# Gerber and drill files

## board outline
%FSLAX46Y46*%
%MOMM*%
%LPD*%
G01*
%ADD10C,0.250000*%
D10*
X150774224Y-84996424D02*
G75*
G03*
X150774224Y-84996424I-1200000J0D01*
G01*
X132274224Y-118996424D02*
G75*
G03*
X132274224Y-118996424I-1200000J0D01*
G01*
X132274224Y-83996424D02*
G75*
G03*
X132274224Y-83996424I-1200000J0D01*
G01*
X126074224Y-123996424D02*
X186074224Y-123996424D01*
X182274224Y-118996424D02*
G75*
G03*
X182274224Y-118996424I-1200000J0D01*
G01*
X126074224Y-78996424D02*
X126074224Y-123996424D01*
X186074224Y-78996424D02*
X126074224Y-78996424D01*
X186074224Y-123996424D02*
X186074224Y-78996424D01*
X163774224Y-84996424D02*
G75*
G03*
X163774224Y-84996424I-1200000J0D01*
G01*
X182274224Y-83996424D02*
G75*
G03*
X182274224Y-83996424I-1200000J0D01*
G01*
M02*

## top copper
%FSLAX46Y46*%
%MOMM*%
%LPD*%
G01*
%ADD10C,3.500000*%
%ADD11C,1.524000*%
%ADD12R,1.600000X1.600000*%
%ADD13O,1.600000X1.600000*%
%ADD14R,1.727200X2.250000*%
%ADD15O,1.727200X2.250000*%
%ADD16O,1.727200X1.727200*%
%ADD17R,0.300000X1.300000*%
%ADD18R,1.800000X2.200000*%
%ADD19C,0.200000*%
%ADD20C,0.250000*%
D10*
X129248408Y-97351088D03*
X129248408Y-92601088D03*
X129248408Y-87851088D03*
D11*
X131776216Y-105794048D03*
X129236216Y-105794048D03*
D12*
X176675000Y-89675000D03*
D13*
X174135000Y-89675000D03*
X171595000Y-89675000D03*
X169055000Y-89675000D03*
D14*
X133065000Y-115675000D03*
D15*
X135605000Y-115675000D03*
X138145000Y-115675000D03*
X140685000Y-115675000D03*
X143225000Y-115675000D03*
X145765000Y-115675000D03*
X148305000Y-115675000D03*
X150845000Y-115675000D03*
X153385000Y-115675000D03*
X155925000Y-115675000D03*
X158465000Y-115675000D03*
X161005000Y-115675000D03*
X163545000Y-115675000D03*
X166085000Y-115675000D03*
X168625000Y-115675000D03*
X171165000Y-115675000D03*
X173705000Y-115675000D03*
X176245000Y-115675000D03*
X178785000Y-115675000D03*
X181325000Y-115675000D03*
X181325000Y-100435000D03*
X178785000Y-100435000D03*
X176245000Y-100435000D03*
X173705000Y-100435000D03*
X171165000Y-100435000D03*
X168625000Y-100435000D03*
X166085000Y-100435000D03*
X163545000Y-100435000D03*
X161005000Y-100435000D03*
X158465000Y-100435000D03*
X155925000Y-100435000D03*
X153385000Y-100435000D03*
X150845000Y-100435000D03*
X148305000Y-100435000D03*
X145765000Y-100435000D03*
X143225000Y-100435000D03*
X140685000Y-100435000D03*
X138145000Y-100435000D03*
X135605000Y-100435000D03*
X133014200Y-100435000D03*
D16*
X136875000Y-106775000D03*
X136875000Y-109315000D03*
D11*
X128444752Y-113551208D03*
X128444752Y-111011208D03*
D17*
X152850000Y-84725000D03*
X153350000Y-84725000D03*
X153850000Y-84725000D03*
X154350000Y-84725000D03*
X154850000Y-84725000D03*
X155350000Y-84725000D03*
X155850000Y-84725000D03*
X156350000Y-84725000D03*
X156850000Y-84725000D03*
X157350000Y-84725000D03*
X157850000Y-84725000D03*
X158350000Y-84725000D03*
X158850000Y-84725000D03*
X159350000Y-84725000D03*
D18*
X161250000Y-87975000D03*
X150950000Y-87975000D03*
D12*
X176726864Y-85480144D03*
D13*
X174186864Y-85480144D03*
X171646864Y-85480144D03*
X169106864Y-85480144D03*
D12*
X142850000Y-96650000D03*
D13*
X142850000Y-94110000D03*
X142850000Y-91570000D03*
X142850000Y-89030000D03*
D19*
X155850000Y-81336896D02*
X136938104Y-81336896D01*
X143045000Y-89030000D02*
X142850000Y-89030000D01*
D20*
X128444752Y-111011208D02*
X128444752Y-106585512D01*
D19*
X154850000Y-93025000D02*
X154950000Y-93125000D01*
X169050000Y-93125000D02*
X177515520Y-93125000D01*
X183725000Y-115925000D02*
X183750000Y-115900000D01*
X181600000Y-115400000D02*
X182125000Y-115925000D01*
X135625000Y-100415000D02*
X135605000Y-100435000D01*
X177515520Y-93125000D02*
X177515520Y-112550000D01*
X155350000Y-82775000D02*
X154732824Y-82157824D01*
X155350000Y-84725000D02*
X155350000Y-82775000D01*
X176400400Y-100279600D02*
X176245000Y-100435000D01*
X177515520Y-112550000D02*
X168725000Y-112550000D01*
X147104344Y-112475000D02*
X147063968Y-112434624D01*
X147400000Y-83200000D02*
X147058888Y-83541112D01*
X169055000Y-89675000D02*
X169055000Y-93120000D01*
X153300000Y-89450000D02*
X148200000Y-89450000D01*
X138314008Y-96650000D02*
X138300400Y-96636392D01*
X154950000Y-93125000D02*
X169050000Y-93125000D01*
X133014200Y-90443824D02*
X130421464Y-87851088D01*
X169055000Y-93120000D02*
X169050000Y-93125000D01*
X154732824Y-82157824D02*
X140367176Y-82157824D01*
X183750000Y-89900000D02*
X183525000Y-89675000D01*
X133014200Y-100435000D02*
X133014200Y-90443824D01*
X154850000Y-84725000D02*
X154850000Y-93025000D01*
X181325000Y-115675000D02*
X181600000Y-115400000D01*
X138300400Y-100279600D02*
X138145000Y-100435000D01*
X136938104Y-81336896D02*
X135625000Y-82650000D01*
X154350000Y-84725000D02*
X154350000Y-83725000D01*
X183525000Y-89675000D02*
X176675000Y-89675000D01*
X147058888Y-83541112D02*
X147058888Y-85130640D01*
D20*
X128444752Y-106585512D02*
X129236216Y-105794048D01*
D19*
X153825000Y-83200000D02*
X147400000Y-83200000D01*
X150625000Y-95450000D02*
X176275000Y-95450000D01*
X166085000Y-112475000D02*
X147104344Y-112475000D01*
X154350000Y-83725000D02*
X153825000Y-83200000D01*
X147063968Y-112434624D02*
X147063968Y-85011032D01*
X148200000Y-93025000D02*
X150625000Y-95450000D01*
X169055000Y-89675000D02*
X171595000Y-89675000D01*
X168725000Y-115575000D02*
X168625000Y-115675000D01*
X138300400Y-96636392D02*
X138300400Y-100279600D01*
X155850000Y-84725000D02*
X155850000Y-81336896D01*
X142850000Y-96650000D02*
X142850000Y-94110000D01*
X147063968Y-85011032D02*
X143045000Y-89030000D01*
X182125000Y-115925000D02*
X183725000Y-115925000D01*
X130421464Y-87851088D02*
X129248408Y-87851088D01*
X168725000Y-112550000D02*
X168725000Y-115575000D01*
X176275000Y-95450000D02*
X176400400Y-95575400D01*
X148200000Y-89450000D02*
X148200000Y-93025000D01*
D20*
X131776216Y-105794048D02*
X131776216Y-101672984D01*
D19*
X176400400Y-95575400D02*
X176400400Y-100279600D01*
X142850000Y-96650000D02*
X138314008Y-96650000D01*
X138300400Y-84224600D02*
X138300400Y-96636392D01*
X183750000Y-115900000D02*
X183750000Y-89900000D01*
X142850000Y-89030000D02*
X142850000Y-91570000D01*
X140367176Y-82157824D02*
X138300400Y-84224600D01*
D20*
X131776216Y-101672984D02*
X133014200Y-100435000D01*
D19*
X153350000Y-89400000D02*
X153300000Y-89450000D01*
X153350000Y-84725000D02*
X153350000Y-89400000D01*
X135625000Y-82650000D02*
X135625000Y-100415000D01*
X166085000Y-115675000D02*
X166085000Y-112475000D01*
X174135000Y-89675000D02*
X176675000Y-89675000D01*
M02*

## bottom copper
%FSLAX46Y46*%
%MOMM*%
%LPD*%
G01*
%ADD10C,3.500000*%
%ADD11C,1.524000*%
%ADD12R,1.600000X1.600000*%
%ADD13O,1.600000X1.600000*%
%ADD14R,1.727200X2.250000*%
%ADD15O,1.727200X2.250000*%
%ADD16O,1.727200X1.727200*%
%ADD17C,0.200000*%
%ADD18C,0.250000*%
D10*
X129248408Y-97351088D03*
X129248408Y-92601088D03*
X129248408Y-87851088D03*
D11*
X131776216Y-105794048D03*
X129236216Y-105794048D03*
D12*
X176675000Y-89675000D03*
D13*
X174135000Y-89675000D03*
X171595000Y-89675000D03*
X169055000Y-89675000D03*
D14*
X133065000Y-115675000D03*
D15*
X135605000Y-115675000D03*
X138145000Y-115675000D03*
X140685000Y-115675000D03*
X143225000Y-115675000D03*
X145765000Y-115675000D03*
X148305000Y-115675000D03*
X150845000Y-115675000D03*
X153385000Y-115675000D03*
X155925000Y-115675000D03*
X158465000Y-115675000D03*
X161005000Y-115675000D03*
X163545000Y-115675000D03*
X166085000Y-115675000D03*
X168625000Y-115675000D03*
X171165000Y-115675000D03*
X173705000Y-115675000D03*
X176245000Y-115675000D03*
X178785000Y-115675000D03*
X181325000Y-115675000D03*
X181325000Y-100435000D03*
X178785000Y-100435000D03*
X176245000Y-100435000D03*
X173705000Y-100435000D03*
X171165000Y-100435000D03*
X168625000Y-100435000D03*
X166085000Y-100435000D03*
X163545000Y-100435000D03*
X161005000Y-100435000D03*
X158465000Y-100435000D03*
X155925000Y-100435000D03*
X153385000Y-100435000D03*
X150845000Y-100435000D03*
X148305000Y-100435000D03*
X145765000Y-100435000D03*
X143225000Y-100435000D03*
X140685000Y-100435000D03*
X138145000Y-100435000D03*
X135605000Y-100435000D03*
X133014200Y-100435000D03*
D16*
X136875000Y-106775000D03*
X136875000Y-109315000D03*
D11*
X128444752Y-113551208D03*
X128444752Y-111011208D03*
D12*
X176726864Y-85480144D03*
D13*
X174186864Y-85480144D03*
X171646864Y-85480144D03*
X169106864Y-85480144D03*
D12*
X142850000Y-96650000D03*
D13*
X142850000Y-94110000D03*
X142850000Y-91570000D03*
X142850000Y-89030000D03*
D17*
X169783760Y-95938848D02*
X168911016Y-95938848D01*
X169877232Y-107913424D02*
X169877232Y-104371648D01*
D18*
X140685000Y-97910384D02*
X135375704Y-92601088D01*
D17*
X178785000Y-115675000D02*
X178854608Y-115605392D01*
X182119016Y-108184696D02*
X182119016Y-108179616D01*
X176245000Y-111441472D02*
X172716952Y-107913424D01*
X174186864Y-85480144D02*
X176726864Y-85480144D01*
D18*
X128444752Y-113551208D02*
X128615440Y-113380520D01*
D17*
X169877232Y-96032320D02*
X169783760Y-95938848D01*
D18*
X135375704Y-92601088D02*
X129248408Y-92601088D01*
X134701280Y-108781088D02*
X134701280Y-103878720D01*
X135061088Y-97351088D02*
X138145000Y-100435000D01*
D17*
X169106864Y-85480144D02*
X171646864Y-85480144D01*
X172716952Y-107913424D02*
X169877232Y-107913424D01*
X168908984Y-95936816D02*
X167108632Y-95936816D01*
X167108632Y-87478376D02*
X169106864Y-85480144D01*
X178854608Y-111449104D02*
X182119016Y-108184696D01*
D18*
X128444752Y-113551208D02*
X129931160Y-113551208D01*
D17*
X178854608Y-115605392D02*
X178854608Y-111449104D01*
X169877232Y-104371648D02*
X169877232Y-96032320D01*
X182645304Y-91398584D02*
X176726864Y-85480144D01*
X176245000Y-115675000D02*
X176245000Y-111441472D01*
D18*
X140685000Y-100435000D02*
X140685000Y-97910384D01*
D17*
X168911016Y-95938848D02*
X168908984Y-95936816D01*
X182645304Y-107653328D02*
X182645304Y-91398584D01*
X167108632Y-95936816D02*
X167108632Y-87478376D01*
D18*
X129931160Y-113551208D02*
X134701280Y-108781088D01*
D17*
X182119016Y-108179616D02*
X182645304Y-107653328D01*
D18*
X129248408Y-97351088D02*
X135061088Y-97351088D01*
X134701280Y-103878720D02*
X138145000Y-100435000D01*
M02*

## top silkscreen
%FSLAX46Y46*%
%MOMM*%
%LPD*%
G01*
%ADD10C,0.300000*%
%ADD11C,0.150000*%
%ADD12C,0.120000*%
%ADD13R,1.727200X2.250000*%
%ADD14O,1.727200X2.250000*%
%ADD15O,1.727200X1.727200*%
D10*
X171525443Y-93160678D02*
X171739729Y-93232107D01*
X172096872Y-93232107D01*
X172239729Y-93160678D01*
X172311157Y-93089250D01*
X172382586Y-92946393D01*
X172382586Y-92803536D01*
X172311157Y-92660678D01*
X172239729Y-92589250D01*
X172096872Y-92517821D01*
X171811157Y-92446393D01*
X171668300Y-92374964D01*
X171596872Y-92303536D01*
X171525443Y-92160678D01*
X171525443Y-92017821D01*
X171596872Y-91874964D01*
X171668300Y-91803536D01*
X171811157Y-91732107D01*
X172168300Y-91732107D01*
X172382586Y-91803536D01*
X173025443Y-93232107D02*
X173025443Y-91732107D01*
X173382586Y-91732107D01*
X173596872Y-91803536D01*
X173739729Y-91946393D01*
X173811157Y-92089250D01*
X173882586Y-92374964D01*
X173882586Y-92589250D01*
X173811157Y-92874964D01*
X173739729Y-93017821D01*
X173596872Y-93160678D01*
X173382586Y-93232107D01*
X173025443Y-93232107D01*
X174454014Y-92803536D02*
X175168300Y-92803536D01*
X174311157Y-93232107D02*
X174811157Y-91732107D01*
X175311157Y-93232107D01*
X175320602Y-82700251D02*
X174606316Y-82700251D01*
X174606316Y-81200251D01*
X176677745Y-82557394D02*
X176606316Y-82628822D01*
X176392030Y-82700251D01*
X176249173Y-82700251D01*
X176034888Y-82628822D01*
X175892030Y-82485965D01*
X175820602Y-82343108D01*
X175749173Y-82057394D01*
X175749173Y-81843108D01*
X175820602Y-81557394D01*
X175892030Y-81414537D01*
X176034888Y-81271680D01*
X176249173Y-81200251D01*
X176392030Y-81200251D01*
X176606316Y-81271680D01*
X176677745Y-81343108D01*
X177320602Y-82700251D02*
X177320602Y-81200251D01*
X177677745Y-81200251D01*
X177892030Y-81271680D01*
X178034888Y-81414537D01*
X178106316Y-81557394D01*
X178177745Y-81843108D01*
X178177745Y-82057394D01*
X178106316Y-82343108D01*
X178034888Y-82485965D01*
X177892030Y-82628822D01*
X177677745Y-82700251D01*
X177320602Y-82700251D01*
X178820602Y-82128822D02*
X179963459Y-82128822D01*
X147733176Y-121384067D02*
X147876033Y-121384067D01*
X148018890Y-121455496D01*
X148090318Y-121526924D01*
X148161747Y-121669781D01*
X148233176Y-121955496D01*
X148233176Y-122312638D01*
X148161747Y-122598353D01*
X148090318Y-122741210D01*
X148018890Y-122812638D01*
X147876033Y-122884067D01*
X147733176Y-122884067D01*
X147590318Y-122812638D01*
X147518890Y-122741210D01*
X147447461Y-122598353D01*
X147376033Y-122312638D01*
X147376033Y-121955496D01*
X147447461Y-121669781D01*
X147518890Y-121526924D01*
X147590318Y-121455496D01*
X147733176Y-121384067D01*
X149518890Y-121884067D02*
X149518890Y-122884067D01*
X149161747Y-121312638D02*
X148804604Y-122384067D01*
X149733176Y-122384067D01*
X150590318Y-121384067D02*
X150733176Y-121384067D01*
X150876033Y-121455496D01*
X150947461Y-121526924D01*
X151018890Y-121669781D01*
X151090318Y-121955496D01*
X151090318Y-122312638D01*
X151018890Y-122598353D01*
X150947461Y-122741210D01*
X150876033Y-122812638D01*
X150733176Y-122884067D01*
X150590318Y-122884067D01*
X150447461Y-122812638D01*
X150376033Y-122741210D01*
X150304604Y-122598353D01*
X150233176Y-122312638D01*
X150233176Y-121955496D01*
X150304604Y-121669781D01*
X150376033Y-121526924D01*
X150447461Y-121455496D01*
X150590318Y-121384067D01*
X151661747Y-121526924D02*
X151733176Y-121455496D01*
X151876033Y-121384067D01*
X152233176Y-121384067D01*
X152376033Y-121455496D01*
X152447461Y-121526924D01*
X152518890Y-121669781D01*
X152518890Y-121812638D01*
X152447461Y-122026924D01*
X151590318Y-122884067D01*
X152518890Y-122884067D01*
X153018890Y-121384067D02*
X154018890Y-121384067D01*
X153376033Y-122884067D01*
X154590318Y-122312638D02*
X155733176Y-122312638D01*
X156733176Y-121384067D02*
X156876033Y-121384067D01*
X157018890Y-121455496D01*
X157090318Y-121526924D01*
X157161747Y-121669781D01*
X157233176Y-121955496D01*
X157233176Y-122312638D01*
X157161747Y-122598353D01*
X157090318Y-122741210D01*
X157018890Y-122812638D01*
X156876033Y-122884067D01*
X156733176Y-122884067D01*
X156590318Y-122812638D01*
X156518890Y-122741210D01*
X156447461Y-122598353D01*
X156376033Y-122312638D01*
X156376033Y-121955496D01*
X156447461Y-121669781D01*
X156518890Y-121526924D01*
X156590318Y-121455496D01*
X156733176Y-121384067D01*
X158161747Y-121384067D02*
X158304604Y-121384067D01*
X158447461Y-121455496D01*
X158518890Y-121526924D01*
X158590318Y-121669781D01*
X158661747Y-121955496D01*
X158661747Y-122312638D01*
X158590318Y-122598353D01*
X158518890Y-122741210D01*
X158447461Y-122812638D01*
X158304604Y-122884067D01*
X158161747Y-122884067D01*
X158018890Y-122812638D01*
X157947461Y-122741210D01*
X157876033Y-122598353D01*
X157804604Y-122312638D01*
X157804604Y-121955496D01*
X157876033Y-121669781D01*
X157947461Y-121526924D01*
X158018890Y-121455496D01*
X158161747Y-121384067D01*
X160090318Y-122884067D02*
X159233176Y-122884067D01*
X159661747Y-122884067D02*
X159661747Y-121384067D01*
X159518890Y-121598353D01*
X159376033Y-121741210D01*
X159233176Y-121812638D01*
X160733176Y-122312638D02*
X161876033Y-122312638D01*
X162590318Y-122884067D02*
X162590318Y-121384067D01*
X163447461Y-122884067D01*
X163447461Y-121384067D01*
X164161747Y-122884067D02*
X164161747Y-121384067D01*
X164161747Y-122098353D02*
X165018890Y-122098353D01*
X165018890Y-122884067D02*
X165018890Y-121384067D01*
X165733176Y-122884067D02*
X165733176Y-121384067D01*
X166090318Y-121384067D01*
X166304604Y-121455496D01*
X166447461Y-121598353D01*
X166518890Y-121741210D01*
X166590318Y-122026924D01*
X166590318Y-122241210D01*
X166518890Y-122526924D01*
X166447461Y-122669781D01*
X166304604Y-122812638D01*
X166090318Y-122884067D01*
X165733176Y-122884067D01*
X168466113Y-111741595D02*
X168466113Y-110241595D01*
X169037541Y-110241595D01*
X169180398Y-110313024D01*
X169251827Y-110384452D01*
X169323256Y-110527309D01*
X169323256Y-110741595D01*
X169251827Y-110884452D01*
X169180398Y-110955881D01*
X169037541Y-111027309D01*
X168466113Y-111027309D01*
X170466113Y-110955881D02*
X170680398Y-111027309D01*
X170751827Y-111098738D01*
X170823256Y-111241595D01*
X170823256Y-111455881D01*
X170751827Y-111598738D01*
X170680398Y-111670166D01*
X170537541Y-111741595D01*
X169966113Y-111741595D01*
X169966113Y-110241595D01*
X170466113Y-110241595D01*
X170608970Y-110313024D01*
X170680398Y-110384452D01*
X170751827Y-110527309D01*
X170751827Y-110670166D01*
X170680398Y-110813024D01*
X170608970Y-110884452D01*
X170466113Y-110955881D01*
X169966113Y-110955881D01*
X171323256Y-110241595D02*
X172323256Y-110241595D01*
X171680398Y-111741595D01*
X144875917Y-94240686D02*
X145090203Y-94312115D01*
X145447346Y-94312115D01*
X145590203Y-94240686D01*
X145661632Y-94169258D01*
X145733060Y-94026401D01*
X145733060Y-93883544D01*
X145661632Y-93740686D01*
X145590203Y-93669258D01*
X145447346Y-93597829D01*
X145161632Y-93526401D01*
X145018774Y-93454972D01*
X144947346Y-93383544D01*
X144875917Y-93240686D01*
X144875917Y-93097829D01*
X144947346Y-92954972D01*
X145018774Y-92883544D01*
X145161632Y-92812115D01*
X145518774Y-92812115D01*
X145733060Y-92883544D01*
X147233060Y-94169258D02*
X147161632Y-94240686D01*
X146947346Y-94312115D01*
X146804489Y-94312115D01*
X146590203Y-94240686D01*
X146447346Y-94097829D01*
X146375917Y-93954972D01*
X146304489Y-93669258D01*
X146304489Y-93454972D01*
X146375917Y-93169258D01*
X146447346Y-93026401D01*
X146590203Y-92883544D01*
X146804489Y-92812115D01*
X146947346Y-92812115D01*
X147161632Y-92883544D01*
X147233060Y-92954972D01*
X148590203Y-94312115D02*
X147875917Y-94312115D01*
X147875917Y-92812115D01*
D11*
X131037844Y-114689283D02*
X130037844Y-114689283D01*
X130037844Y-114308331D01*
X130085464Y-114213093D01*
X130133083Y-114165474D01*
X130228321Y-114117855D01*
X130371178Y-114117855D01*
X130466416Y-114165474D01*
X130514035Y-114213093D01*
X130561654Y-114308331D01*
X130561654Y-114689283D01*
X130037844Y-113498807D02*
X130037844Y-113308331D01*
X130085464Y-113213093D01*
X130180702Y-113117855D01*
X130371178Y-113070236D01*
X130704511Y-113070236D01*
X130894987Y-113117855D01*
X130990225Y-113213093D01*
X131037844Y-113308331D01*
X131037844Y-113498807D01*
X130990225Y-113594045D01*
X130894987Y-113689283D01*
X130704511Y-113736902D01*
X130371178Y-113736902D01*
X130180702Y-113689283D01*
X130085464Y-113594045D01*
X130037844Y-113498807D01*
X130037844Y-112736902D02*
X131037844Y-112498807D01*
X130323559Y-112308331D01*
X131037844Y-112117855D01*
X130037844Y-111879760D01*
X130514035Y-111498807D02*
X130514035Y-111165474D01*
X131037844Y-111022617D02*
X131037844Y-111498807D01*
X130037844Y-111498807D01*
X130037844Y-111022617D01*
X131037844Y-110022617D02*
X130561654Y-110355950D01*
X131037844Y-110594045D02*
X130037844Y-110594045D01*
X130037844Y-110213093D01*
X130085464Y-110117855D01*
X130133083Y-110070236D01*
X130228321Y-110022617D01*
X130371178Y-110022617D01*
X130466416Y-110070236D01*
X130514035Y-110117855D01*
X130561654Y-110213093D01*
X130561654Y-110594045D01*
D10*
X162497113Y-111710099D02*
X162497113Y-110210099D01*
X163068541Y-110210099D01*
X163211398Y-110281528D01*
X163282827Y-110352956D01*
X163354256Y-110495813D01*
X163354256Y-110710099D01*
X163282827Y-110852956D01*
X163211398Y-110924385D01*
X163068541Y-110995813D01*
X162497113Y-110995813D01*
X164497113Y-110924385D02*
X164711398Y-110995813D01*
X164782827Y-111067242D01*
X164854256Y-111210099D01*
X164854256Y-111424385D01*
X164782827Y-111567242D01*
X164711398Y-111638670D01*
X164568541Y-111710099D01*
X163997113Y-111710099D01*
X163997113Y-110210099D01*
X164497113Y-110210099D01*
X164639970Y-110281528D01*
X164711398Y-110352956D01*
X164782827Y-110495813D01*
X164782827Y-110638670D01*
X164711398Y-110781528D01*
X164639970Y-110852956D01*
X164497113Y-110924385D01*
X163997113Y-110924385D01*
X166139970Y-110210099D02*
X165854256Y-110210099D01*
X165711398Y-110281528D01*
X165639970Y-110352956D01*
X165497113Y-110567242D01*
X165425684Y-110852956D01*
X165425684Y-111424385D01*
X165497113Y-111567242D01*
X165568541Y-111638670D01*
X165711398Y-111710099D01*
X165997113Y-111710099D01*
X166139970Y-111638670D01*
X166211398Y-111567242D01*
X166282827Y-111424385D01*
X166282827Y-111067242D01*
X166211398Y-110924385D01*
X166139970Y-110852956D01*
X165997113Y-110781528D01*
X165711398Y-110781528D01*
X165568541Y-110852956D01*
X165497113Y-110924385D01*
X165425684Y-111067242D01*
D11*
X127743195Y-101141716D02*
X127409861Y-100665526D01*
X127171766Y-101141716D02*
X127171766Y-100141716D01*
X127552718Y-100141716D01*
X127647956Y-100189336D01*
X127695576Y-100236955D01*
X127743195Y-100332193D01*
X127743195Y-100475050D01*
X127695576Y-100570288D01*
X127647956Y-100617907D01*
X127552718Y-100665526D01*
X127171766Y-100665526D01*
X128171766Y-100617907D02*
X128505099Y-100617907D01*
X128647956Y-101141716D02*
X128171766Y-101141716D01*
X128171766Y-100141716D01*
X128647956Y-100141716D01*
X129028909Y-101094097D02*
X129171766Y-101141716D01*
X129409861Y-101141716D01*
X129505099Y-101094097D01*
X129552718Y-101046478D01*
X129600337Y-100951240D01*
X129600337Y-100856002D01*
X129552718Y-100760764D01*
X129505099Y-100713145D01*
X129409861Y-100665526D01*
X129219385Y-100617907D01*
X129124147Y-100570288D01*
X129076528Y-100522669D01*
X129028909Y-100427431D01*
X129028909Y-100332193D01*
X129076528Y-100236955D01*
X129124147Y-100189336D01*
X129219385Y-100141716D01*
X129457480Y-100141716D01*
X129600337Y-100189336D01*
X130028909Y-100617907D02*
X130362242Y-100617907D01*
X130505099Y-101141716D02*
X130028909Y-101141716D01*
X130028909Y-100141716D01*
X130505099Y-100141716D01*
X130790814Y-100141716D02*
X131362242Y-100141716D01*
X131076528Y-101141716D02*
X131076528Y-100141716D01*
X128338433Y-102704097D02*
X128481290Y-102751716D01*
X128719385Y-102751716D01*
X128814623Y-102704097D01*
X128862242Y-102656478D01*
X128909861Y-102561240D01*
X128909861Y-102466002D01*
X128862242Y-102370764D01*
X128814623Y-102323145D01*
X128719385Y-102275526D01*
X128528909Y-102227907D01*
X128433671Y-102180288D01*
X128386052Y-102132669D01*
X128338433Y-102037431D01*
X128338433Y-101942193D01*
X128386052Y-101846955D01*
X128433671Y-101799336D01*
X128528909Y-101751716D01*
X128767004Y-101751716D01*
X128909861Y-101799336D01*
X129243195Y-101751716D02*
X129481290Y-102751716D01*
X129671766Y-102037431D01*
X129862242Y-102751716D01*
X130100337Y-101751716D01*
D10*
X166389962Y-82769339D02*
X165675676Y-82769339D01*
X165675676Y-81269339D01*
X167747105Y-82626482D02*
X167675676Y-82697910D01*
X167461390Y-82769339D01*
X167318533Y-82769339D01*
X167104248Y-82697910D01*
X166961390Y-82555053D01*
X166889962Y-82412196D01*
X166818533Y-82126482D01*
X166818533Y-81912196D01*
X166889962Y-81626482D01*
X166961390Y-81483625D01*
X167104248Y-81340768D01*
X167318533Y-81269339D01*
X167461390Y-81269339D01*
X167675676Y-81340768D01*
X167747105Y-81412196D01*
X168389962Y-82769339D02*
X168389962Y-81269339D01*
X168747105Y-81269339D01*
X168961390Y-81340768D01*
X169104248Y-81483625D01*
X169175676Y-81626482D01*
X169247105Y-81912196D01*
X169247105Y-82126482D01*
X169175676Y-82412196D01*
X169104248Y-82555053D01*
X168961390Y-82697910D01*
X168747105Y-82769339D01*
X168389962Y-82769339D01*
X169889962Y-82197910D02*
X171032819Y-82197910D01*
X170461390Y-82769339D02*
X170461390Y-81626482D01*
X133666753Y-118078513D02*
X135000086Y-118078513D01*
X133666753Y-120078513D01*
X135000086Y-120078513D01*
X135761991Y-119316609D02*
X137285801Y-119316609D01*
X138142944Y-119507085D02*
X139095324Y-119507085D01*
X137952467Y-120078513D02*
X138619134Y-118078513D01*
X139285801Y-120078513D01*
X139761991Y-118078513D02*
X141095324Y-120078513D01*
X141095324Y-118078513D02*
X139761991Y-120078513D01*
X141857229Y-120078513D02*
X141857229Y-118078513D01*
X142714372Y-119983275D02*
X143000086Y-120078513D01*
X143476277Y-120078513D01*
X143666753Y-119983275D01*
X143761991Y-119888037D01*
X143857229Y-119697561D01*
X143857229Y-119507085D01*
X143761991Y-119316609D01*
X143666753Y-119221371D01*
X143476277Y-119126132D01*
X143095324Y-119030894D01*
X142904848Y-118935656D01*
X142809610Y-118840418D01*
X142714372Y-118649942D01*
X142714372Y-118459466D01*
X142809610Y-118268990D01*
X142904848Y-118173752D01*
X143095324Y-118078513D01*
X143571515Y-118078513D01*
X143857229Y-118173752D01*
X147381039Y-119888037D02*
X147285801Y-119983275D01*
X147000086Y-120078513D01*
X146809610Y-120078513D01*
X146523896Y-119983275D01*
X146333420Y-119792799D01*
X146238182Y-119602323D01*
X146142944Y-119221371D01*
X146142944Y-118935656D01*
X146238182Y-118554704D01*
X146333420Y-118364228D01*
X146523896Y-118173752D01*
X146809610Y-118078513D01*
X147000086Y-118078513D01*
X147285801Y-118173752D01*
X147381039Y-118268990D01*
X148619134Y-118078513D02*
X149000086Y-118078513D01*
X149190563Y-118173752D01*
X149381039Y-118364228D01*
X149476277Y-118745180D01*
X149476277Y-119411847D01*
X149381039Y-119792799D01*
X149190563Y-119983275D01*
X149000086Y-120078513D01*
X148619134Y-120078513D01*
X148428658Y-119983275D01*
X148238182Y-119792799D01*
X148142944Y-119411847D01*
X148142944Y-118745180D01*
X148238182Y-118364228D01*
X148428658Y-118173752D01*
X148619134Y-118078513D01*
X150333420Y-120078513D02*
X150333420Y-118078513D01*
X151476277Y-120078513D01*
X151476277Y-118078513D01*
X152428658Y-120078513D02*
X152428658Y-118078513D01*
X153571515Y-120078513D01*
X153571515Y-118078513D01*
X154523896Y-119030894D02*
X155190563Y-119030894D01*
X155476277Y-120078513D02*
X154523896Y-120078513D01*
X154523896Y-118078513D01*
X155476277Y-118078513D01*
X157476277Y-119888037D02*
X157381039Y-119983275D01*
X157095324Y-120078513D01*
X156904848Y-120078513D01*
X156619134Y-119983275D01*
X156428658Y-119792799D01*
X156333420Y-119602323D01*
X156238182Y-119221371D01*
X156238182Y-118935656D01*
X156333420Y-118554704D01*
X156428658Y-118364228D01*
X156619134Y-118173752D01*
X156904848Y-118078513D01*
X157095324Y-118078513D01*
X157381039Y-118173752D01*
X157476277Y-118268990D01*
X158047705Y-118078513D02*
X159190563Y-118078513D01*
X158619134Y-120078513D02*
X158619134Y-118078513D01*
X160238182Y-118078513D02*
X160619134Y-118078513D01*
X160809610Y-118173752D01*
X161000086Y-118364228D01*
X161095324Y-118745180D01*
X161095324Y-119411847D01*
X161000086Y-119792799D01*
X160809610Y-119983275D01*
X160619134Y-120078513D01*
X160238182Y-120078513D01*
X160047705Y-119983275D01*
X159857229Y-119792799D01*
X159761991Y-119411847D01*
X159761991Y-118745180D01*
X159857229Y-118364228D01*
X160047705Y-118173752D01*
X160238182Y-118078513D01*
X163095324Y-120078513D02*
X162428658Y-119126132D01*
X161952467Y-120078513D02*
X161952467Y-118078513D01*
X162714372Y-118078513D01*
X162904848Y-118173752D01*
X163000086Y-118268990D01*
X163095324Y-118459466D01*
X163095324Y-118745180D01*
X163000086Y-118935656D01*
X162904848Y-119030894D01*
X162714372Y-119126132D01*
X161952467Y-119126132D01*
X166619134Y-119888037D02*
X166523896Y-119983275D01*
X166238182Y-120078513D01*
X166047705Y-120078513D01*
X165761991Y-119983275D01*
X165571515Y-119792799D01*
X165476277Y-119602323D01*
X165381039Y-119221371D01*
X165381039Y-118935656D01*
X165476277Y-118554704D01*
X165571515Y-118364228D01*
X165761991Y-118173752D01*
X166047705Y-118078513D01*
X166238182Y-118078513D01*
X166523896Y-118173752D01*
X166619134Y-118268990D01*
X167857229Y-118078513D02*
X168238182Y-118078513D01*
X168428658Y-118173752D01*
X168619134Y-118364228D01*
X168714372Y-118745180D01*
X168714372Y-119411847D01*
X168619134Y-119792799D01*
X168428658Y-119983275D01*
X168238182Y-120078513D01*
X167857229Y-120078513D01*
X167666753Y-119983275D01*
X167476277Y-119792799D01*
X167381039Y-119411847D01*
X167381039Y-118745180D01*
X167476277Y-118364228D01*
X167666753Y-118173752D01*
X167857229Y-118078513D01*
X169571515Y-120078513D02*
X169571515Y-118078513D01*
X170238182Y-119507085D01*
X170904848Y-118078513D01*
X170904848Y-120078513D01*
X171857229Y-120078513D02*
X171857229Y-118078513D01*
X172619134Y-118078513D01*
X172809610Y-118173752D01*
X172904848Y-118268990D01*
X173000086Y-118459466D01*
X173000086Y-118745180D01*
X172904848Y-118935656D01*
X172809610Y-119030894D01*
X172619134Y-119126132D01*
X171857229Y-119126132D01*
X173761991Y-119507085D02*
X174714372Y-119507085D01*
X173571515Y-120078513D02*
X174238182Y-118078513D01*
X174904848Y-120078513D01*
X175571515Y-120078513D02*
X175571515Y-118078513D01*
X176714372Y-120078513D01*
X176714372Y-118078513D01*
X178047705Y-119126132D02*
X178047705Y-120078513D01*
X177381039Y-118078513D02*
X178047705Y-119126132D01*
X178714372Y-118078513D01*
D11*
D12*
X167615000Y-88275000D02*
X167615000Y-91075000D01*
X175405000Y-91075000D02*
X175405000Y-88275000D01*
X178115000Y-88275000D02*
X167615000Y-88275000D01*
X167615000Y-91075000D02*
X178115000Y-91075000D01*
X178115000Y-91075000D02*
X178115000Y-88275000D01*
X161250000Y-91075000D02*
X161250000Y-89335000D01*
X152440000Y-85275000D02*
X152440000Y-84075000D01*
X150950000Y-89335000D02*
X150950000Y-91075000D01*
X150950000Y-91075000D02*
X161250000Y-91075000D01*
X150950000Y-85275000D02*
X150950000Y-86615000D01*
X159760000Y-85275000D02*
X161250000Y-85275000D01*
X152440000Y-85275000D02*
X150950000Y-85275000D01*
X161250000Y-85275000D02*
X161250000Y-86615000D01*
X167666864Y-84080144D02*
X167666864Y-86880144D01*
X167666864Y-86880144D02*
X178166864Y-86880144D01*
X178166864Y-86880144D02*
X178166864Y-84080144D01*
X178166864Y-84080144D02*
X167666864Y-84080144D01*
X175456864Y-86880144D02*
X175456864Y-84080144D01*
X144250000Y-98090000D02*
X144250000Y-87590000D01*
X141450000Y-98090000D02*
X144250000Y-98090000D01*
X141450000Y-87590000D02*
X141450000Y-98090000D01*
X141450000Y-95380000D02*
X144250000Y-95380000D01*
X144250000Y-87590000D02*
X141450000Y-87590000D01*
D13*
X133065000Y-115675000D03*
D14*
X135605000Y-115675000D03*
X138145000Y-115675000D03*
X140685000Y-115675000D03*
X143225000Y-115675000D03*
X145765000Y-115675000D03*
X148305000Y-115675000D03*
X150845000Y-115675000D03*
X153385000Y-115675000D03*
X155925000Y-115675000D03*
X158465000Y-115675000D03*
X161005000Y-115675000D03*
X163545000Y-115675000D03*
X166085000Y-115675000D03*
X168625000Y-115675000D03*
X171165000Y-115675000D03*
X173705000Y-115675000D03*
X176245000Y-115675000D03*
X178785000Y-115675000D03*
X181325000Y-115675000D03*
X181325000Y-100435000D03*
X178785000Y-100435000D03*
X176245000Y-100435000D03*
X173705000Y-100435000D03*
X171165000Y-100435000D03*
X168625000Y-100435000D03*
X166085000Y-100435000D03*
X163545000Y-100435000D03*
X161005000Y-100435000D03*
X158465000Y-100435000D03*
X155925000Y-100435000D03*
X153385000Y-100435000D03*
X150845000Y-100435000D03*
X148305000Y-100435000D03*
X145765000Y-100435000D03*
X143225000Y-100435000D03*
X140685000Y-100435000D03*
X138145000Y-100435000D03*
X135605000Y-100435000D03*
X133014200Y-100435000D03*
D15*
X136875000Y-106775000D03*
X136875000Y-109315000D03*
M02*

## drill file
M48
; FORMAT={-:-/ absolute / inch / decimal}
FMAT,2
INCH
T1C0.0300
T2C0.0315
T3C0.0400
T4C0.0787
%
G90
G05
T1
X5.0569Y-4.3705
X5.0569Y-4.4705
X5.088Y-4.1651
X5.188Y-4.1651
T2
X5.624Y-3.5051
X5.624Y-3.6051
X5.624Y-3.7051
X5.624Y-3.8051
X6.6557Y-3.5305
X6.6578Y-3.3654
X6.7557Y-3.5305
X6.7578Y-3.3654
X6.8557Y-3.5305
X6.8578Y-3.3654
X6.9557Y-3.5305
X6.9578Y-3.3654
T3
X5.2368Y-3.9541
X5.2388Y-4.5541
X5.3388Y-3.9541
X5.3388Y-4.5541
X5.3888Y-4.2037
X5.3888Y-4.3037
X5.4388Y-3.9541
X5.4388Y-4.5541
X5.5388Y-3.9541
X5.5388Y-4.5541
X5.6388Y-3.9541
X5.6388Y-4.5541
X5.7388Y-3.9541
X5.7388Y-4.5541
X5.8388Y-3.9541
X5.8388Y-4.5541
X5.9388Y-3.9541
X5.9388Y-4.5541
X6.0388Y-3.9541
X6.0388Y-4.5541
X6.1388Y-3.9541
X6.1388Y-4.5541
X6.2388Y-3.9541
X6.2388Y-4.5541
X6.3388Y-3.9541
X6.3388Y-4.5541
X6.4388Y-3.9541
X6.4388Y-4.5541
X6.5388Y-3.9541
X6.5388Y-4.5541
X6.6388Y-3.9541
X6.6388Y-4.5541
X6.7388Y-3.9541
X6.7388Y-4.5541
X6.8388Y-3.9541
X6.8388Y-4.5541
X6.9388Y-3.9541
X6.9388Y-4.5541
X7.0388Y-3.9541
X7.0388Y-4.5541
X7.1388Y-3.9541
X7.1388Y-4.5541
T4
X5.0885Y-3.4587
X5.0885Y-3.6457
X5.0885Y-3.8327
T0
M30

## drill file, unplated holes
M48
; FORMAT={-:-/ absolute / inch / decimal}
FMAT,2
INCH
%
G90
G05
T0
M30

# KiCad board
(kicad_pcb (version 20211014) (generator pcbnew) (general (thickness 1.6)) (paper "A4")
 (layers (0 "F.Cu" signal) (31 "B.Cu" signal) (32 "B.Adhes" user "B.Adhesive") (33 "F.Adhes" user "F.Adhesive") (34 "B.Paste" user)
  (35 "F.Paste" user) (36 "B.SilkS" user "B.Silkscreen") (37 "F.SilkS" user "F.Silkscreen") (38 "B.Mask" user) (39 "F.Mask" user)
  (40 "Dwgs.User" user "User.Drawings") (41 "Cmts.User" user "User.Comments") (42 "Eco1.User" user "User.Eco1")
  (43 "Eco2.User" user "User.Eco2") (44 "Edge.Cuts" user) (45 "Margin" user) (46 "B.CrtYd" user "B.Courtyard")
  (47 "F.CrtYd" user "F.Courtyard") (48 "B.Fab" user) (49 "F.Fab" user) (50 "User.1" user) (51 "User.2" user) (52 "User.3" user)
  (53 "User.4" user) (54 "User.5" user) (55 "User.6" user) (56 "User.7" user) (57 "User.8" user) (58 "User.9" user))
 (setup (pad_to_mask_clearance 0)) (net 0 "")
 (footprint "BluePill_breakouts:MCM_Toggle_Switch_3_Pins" (layer "F.Cu") (at 129.248408 97.351088 90)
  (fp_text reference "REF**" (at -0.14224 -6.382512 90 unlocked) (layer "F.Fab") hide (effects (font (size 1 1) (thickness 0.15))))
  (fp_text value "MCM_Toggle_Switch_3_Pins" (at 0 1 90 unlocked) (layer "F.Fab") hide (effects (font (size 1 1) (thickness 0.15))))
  (pad "1" thru_hole circle (at 0 0 90) (size 3.5 3.5) (drill 2) (layers *.Cu *.Mask))
  (pad "2" thru_hole circle (at 4.75 0 90) (size 3.5 3.5) (drill 2) (layers *.Cu *.Mask))
  (pad "3" thru_hole circle (at 9.5 0 90) (size 3.5 3.5) (drill 2) (layers *.Cu *.Mask)))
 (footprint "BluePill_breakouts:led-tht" (layer "F.Cu") (at 131.776216 105.794048 180)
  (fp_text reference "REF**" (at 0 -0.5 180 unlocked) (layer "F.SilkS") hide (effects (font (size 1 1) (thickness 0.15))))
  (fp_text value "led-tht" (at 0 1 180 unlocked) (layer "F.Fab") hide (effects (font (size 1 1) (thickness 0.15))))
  (pad "1" thru_hole circle (at 0 0 180) (size 1.524 1.524) (drill 0.762) (layers *.Cu *.Mask))
  (pad "2" thru_hole circle (at 2.54 0 180) (size 1.524 1.524) (drill 0.762) (layers *.Cu *.Mask)))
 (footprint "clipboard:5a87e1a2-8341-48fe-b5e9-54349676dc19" (layer "F.Cu") (at 176.675 89.675 180)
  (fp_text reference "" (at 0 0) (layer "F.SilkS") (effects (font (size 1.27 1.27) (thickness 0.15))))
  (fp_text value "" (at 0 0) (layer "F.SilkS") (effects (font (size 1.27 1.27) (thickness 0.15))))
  (fp_line (start 9.06 1.4) (end 9.06 -1.4) (layer "F.SilkS") (width 0.12))
  (fp_line (start 1.27 -1.4) (end 1.27 1.4) (layer "F.SilkS") (width 0.12))
  (fp_line (start -1.44 1.4) (end 9.06 1.4) (layer "F.SilkS") (width 0.12))
  (fp_line (start 9.06 -1.4) (end -1.44 -1.4) (layer "F.SilkS") (width 0.12))
  (fp_line (start -1.44 -1.4) (end -1.44 1.4) (layer "F.SilkS") (width 0.12))
  (pad "1" thru_hole rect (at 0 0 180) (size 1.6 1.6) (drill 0.8) (layers *.Cu *.Mask))
  (pad "2" thru_hole oval (at 2.54 0 180) (size 1.6 1.6) (drill 0.8) (layers *.Cu *.Mask))
  (pad "3" thru_hole oval (at 5.08 0 180) (size 1.6 1.6) (drill 0.8) (layers *.Cu *.Mask))
  (pad "4" thru_hole oval (at 7.62 0 180) (size 1.6 1.6) (drill 0.8) (layers *.Cu *.Mask)))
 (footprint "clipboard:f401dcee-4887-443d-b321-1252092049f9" (layer "F.Cu") (at 133.0142 100.435 90)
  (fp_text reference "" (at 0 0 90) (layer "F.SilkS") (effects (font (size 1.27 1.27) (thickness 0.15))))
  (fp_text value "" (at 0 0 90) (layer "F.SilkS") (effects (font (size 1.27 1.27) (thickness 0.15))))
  (pad "1" thru_hole rect (at -15.24 0.0508) (size 1.7272 2.25) (drill 1.016) (layers *.Cu *.Mask "F.SilkS"))
  (pad "2" thru_hole oval (at -15.24 2.5908) (size 1.7272 2.25) (drill 1.016) (layers *.Cu *.Mask "F.SilkS"))
  (pad "3" thru_hole oval (at -15.24 5.1308) (size 1.7272 2.25) (drill 1.016) (layers *.Cu *.Mask "F.SilkS"))
  (pad "4" thru_hole oval (at -15.24 7.6708) (size 1.7272 2.25) (drill 1.016) (layers *.Cu *.Mask "F.SilkS"))
  (pad "5" thru_hole oval (at -15.24 10.2108) (size 1.7272 2.25) (drill 1.016) (layers *.Cu *.Mask "F.SilkS"))
  (pad "6" thru_hole oval (at -15.24 12.7508) (size 1.7272 2.25) (drill 1.016) (layers *.Cu *.Mask "F.SilkS"))
  (pad "7" thru_hole oval (at -15.24 15.2908) (size 1.7272 2.25) (drill 1.016) (layers *.Cu *.Mask "F.SilkS"))
  (pad "8" thru_hole oval (at -15.24 17.8308) (size 1.7272 2.25) (drill 1.016) (layers *.Cu *.Mask "F.SilkS"))
  (pad "9" thru_hole oval (at -15.24 20.3708) (size 1.7272 2.25) (drill 1.016) (layers *.Cu *.Mask "F.SilkS"))
  (pad "10" thru_hole oval (at -15.24 22.9108) (size 1.7272 2.25) (drill 1.016) (layers *.Cu *.Mask "F.SilkS"))
  (pad "11" thru_hole oval (at -15.24 25.4508) (size 1.7272 2.25) (drill 1.016) (layers *.Cu *.Mask "F.SilkS"))
  (pad "12" thru_hole oval (at -15.24 27.9908) (size 1.7272 2.25) (drill 1.016) (layers *.Cu *.Mask "F.SilkS"))
  (pad "13" thru_hole oval (at -15.24 30.5308) (size 1.7272 2.25) (drill 1.016) (layers *.Cu *.Mask "F.SilkS"))
  (pad "14" thru_hole oval (at -15.24 33.0708) (size 1.7272 2.25) (drill 1.016) (layers *.Cu *.Mask "F.SilkS"))
  (pad "15" thru_hole oval (at -15.24 35.6108) (size 1.7272 2.25) (drill 1.016) (layers *.Cu *.Mask "F.SilkS"))
  (pad "16" thru_hole oval (at -15.24 38.1508) (size 1.7272 2.25) (drill 1.016) (layers *.Cu *.Mask "F.SilkS"))
  (pad "17" thru_hole oval (at -15.24 40.6908) (size 1.7272 2.25) (drill 1.016) (layers *.Cu *.Mask "F.SilkS"))
  (pad "18" thru_hole oval (at -15.24 43.2308) (size 1.7272 2.25) (drill 1.016) (layers *.Cu *.Mask "F.SilkS"))
  (pad "19" thru_hole oval (at -15.24 45.7708) (size 1.7272 2.25) (drill 1.016) (layers *.Cu *.Mask "F.SilkS"))
  (pad "20" thru_hole oval (at -15.24 48.3108) (size 1.7272 2.25) (drill 1.016) (layers *.Cu *.Mask "F.SilkS"))
  (pad "21" thru_hole oval (at 0 48.3108 180) (size 1.7272 2.25) (drill 1.016) (layers *.Cu *.Mask "F.SilkS"))
  (pad "22" thru_hole oval (at 0 45.7708 180) (size 1.7272 2.25) (drill 1.016) (layers *.Cu *.Mask "F.SilkS"))
  (pad "23" thru_hole oval (at 0 43.2308 180) (size 1.7272 2.25) (drill 1.016) (layers *.Cu *.Mask "F.SilkS"))
  (pad "24" thru_hole oval (at 0 40.6908 180) (size 1.7272 2.25) (drill 1.016) (layers *.Cu *.Mask "F.SilkS"))
  (pad "25" thru_hole oval (at 0 38.1508 180) (size 1.7272 2.25) (drill 1.016) (layers *.Cu *.Mask "F.SilkS"))
  (pad "26" thru_hole oval (at 0 35.6108 180) (size 1.7272 2.25) (drill 1.016) (layers *.Cu *.Mask "F.SilkS"))
  (pad "27" thru_hole oval (at 0 33.0708 180) (size 1.7272 2.25) (drill 1.016) (layers *.Cu *.Mask "F.SilkS"))
  (pad "28" thru_hole oval (at 0 30.5308 180) (size 1.7272 2.25) (drill 1.016) (layers *.Cu *.Mask "F.SilkS"))
  (pad "29" thru_hole oval (at 0 27.9908 180) (size 1.7272 2.25) (drill 1.016) (layers *.Cu *.Mask "F.SilkS"))
  (pad "30" thru_hole oval (at 0 25.4508 180) (size 1.7272 2.25) (drill 1.016) (layers *.Cu *.Mask "F.SilkS"))
  (pad "31" thru_hole oval (at 0 22.9108 180) (size 1.7272 2.25) (drill 1.016) (layers *.Cu *.Mask "F.SilkS"))
  (pad "32" thru_hole oval (at 0 20.3708 180) (size 1.7272 2.25) (drill 1.016) (layers *.Cu *.Mask "F.SilkS"))
  (pad "33" thru_hole oval (at 0 17.8308 180) (size 1.7272 2.25) (drill 1.016) (layers *.Cu *.Mask "F.SilkS"))
  (pad "34" thru_hole oval (at 0 15.2908 180) (size 1.7272 2.25) (drill 1.016) (layers *.Cu *.Mask "F.SilkS"))
  (pad "35" thru_hole oval (at 0 12.7508 180) (size 1.7272 2.25) (drill 1.016) (layers *.Cu *.Mask "F.SilkS"))
  (pad "36" thru_hole oval (at 0 10.2108 180) (size 1.7272 2.25) (drill 1.016) (layers *.Cu *.Mask "F.SilkS"))
  (pad "37" thru_hole oval (at 0 7.6708 180) (size 1.7272 2.25) (drill 1.016) (layers *.Cu *.Mask "F.SilkS"))
  (pad "38" thru_hole oval (at 0 5.1308 180) (size 1.7272 2.25) (drill 1.016) (layers *.Cu *.Mask "F.SilkS"))
  (pad "39" thru_hole oval (at 0 2.5908 180) (size 1.7272 2.25) (drill 1.016) (layers *.Cu *.Mask "F.SilkS"))
  (pad "40" thru_hole oval (at 0 0 180) (size 1.7272 2.25) (drill 1.016) (layers *.Cu *.Mask "F.SilkS"))
  (pad "41" thru_hole oval (at -6.34 3.8608 180) (size 1.7272 1.7272) (drill 1.016) (layers *.Cu *.Mask "F.SilkS"))
  (pad "42" thru_hole oval (at -8.88 3.8608 180) (size 1.7272 1.7272) (drill 1.016) (layers *.Cu *.Mask "F.SilkS")))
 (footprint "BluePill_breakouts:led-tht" (layer "F.Cu") (at 128.444752 113.551208 90)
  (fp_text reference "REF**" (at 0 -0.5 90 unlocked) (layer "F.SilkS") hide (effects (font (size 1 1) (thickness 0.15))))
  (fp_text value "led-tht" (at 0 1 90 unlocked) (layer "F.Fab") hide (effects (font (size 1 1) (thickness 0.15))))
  (pad "1" thru_hole circle (at 0 0 90) (size 1.524 1.524) (drill 0.762) (layers *.Cu *.Mask))
  (pad "2" thru_hole circle (at 2.54 0 90) (size 1.524 1.524) (drill 0.762) (layers *.Cu *.Mask)))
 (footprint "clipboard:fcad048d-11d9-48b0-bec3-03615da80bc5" (layer "F.Cu") (at 156.1 85.375)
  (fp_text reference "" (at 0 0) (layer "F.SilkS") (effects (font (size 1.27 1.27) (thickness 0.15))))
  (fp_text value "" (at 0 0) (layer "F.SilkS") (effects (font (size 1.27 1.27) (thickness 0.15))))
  (fp_line (start 5.15 5.7) (end 5.15 3.96) (layer "F.SilkS") (width 0.12))
  (fp_line (start -3.66 -0.1) (end -3.66 -1.3) (layer "F.SilkS") (width 0.12))
  (fp_line (start -5.15 3.96) (end -5.15 5.7) (layer "F.SilkS") (width 0.12))
  (fp_line (start -5.15 5.7) (end 5.15 5.7) (layer "F.SilkS") (width 0.12))
  (fp_line (start -5.15 -0.1) (end -5.15 1.24) (layer "F.SilkS") (width 0.12))
  (fp_line (start 3.66 -0.1) (end 5.15 -0.1) (layer "F.SilkS") (width 0.12))
  (fp_line (start -3.66 -0.1) (end -5.15 -0.1) (layer "F.SilkS") (width 0.12))
  (fp_line (start 5.15 -0.1) (end 5.15 1.24) (layer "F.SilkS") (width 0.12))
  (pad "1" smd rect (at -3.25 -0.65) (size 0.3 1.3) (layers "F.Cu" "F.Paste" "F.Mask"))
  (pad "2" smd rect (at -2.75 -0.65) (size 0.3 1.3) (layers "F.Cu" "F.Paste" "F.Mask"))
  (pad "3" smd rect (at -2.25 -0.65) (size 0.3 1.3) (layers "F.Cu" "F.Paste" "F.Mask"))
  (pad "4" smd rect (at -1.75 -0.65) (size 0.3 1.3) (layers "F.Cu" "F.Paste" "F.Mask"))
  (pad "5" smd rect (at -1.25 -0.65) (size 0.3 1.3) (layers "F.Cu" "F.Paste" "F.Mask"))
  (pad "6" smd rect (at -0.75 -0.65) (size 0.3 1.3) (layers "F.Cu" "F.Paste" "F.Mask"))
  (pad "7" smd rect (at -0.25 -0.65) (size 0.3 1.3) (layers "F.Cu" "F.Paste" "F.Mask"))
  (pad "8" smd rect (at 0.25 -0.65) (size 0.3 1.3) (layers "F.Cu" "F.Paste" "F.Mask"))
  (pad "9" smd rect (at 0.75 -0.65) (size 0.3 1.3) (layers "F.Cu" "F.Paste" "F.Mask"))
  (pad "10" smd rect (at 1.25 -0.65) (size 0.3 1.3) (layers "F.Cu" "F.Paste" "F.Mask"))
  (pad "11" smd rect (at 1.75 -0.65) (size 0.3 1.3) (layers "F.Cu" "F.Paste" "F.Mask"))
  (pad "12" smd rect (at 2.25 -0.65) (size 0.3 1.3) (layers "F.Cu" "F.Paste" "F.Mask"))
  (pad "13" smd rect (at 2.75 -0.65) (size 0.3 1.3) (layers "F.Cu" "F.Paste" "F.Mask"))
  (pad "14" smd rect (at 3.25 -0.65) (size 0.3 1.3) (layers "F.Cu" "F.Paste" "F.Mask"))
  (pad "MP" smd rect (at 5.15 2.6) (size 1.8 2.2) (layers "F.Cu" "F.Paste" "F.Mask"))
  (pad "MP" smd rect (at -5.15 2.6) (size 1.8 2.2) (layers "F.Cu" "F.Paste" "F.Mask")))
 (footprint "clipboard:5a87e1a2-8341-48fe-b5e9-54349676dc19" (layer "F.Cu") (at 176.726864 85.480144 180)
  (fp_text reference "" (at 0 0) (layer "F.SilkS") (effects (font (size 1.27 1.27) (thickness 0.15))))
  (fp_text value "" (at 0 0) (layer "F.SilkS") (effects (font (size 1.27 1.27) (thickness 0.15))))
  (fp_line (start 9.06 1.4) (end 9.06 -1.4) (layer "F.SilkS") (width 0.12))
  (fp_line (start 9.06 -1.4) (end -1.44 -1.4) (layer "F.SilkS") (width 0.12))
  (fp_line (start -1.44 -1.4) (end -1.44 1.4) (layer "F.SilkS") (width 0.12))
  (fp_line (start -1.44 1.4) (end 9.06 1.4) (layer "F.SilkS") (width 0.12))
  (fp_line (start 1.27 -1.4) (end 1.27 1.4) (layer "F.SilkS") (width 0.12))
  (pad "1" thru_hole rect (at 0 0 180) (size 1.6 1.6) (drill 0.8) (layers *.Cu *.Mask))
  (pad "2" thru_hole oval (at 2.54 0 180) (size 1.6 1.6) (drill 0.8) (layers *.Cu *.Mask))
  (pad "3" thru_hole oval (at 5.08 0 180) (size 1.6 1.6) (drill 0.8) (layers *.Cu *.Mask))
  (pad "4" thru_hole oval (at 7.62 0 180) (size 1.6 1.6) (drill 0.8) (layers *.Cu *.Mask)))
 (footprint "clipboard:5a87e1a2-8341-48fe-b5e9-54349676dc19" (layer "F.Cu") (at 142.85 96.65 90)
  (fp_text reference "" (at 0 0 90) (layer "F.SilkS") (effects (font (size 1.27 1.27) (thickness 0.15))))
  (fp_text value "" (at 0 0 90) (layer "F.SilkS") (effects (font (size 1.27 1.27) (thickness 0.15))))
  (fp_line (start -1.44 1.4) (end 9.06 1.4) (layer "F.SilkS") (width 0.12))
  (fp_line (start -1.44 -1.4) (end -1.44 1.4) (layer "F.SilkS") (width 0.12))
  (fp_line (start 9.06 -1.4) (end -1.44 -1.4) (layer "F.SilkS") (width 0.12))
  (fp_line (start 1.27 -1.4) (end 1.27 1.4) (layer "F.SilkS") (width 0.12))
  (fp_line (start 9.06 1.4) (end 9.06 -1.4) (layer "F.SilkS") (width 0.12))
  (pad "1" thru_hole rect (at 0 0 90) (size 1.6 1.6) (drill 0.8) (layers *.Cu *.Mask))
  (pad "2" thru_hole oval (at 2.54 0 90) (size 1.6 1.6) (drill 0.8) (layers *.Cu *.Mask))
  (pad "3" thru_hole oval (at 5.08 0 90) (size 1.6 1.6) (drill 0.8) (layers *.Cu *.Mask))
  (pad "4" thru_hole oval (at 7.62 0 90) (size 1.6 1.6) (drill 0.8) (layers *.Cu *.Mask)))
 (gr_circle (center 149.574224 84.996424) (end 150.774224 84.996424) (layer "Edge.Cuts") (width 0.25) (fill none))
 (gr_circle (center 131.074224 118.996424) (end 132.274224 118.996424) (layer "Edge.Cuts") (width 0.25) (fill none))
 (gr_circle (center 131.074224 83.996424) (end 132.274224 83.996424) (layer "Edge.Cuts") (width 0.25) (fill none))
 (gr_line (start 126.074224 123.996424) (end 186.074224 123.996424) (layer "Edge.Cuts") (width 0.25))
 (gr_circle (center 181.074224 118.996424) (end 182.274224 118.996424) (layer "Edge.Cuts") (width 0.25) (fill none))
 (gr_line (start 126.074224 78.996424) (end 126.074224 123.996424) (layer "Edge.Cuts") (width 0.25))
 (gr_line (start 186.074224 78.996424) (end 126.074224 78.996424) (layer "Edge.Cuts") (width 0.25))
 (gr_line (start 186.074224 123.996424) (end 186.074224 78.996424) (layer "Edge.Cuts") (width 0.25))
 (gr_circle (center 162.574224 84.996424) (end 163.774224 84.996424) (layer "Edge.Cuts") (width 0.25) (fill none))
 (gr_circle (center 181.074224 83.996424) (end 182.274224 83.996424) (layer "Edge.Cuts") (width 0.25) (fill none))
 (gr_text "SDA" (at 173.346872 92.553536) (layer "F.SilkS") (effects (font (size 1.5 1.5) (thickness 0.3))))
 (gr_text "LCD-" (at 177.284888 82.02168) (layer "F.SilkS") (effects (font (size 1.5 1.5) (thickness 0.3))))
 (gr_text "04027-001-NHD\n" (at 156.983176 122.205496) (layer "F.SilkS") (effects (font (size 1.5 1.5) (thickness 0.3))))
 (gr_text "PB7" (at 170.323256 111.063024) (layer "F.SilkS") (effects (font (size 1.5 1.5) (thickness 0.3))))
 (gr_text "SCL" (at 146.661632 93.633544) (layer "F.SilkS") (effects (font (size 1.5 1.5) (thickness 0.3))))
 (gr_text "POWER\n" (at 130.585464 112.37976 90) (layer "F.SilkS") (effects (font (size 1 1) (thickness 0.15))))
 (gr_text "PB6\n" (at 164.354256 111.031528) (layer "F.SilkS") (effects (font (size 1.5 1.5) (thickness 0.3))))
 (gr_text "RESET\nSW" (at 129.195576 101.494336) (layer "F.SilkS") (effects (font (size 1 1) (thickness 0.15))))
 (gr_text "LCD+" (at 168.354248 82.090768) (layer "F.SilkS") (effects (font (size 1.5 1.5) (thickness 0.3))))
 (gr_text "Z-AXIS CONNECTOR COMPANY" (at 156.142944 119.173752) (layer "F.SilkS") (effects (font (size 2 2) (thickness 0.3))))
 (segment (start 155.85 81.336896) (end 136.938104 81.336896) (width 0.2) (layer "F.Cu") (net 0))
 (segment (start 143.045 89.03) (end 142.85 89.03) (width 0.2) (layer "F.Cu") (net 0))
 (segment (start 128.444752 111.011208) (end 128.444752 106.585512) (width 0.25) (layer "F.Cu") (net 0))
 (segment (start 154.85 93.025) (end 154.95 93.125) (width 0.2) (layer "F.Cu") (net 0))
 (segment (start 169.05 93.125) (end 177.51552 93.125) (width 0.2) (layer "F.Cu") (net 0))
 (segment (start 183.725 115.925) (end 183.75 115.9) (width 0.2) (layer "F.Cu") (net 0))
 (segment (start 181.6 115.4) (end 182.125 115.925) (width 0.2) (layer "F.Cu") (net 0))
 (segment (start 135.625 100.415) (end 135.605 100.435) (width 0.2) (layer "F.Cu") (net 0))
 (segment (start 177.51552 93.125) (end 177.51552 112.55) (width 0.2) (layer "F.Cu") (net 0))
 (segment (start 155.35 82.775) (end 154.732824 82.157824) (width 0.2) (layer "F.Cu") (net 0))
 (segment (start 155.35 84.725) (end 155.35 82.775) (width 0.2) (layer "F.Cu") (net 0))
 (segment (start 176.4004 100.2796) (end 176.245 100.435) (width 0.2) (layer "F.Cu") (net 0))
 (segment (start 177.51552 112.55) (end 168.725 112.55) (width 0.2) (layer "F.Cu") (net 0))
 (segment (start 147.104344 112.475) (end 147.063968 112.434624) (width 0.2) (layer "F.Cu") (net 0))
 (segment (start 147.4 83.2) (end 147.058888 83.541112) (width 0.2) (layer "F.Cu") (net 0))
 (segment (start 169.055 89.675) (end 169.055 93.12) (width 0.2) (layer "F.Cu") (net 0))
 (segment (start 153.3 89.45) (end 148.2 89.45) (width 0.2) (layer "F.Cu") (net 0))
 (segment (start 138.314008 96.65) (end 138.3004 96.636392) (width 0.2) (layer "F.Cu") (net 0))
 (segment (start 154.95 93.125) (end 169.05 93.125) (width 0.2) (layer "F.Cu") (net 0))
 (segment (start 133.0142 90.443824) (end 130.421464 87.851088) (width 0.2) (layer "F.Cu") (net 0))
 (segment (start 169.055 93.12) (end 169.05 93.125) (width 0.2) (layer "F.Cu") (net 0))
 (segment (start 154.732824 82.157824) (end 140.367176 82.157824) (width 0.2) (layer "F.Cu") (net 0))
 (segment (start 183.75 89.9) (end 183.525 89.675) (width 0.2) (layer "F.Cu") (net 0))
 (segment (start 133.0142 100.435) (end 133.0142 90.443824) (width 0.2) (layer "F.Cu") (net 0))
 (segment (start 154.85 84.725) (end 154.85 93.025) (width 0.2) (layer "F.Cu") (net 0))
 (segment (start 181.325 115.675) (end 181.6 115.4) (width 0.2) (layer "F.Cu") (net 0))
 (segment (start 138.3004 100.2796) (end 138.145 100.435) (width 0.2) (layer "F.Cu") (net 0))
 (segment (start 136.938104 81.336896) (end 135.625 82.65) (width 0.2) (layer "F.Cu") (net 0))
 (segment (start 154.35 84.725) (end 154.35 83.725) (width 0.2) (layer "F.Cu") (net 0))
 (segment (start 183.525 89.675) (end 176.675 89.675) (width 0.2) (layer "F.Cu") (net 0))
 (segment (start 147.058888 83.541112) (end 147.058888 85.13064) (width 0.2) (layer "F.Cu") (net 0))
 (segment (start 128.444752 106.585512) (end 129.236216 105.794048) (width 0.25) (layer "F.Cu") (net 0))
 (segment (start 153.825 83.2) (end 147.4 83.2) (width 0.2) (layer "F.Cu") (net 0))
 (segment (start 150.625 95.45) (end 176.275 95.45) (width 0.2) (layer "F.Cu") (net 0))
 (segment (start 166.085 112.475) (end 147.104344 112.475) (width 0.2) (layer "F.Cu") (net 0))
 (segment (start 154.35 83.725) (end 153.825 83.2) (width 0.2) (layer "F.Cu") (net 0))
 (segment (start 147.063968 112.434624) (end 147.063968 85.011032) (width 0.2) (layer "F.Cu") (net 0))
 (segment (start 148.2 93.025) (end 150.625 95.45) (width 0.2) (layer "F.Cu") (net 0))
 (segment (start 169.055 89.675) (end 171.595 89.675) (width 0.2) (layer "F.Cu") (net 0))
 (segment (start 168.725 115.575) (end 168.625 115.675) (width 0.2) (layer "F.Cu") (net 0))
 (segment (start 138.3004 96.636392) (end 138.3004 100.2796) (width 0.2) (layer "F.Cu") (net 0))
 (segment (start 155.85 84.725) (end 155.85 81.336896) (width 0.2) (layer "F.Cu") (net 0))
 (segment (start 142.85 96.65) (end 142.85 94.11) (width 0.2) (layer "F.Cu") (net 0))
 (segment (start 147.063968 85.011032) (end 143.045 89.03) (width 0.2) (layer "F.Cu") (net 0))
 (segment (start 182.125 115.925) (end 183.725 115.925) (width 0.2) (layer "F.Cu") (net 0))
 (segment (start 130.421464 87.851088) (end 129.248408 87.851088) (width 0.2) (layer "F.Cu") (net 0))
 (segment (start 168.725 112.55) (end 168.725 115.575) (width 0.2) (layer "F.Cu") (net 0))
 (segment (start 176.275 95.45) (end 176.4004 95.5754) (width 0.2) (layer "F.Cu") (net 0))
 (segment (start 148.2 89.45) (end 148.2 93.025) (width 0.2) (layer "F.Cu") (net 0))
 (segment (start 131.776216 105.794048) (end 131.776216 101.672984) (width 0.25) (layer "F.Cu") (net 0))
 (segment (start 176.4004 95.5754) (end 176.4004 100.2796) (width 0.2) (layer "F.Cu") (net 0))
 (segment (start 142.85 96.65) (end 138.314008 96.65) (width 0.2) (layer "F.Cu") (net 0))
 (segment (start 138.3004 84.2246) (end 138.3004 96.636392) (width 0.2) (layer "F.Cu") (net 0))
 (segment (start 183.75 115.9) (end 183.75 89.9) (width 0.2) (layer "F.Cu") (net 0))
 (segment (start 142.85 89.03) (end 142.85 91.57) (width 0.2) (layer "F.Cu") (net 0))
 (segment (start 140.367176 82.157824) (end 138.3004 84.2246) (width 0.2) (layer "F.Cu") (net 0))
 (segment (start 131.776216 101.672984) (end 133.0142 100.435) (width 0.25) (layer "F.Cu") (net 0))
 (segment (start 153.35 89.4) (end 153.3 89.45) (width 0.2) (layer "F.Cu") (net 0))
 (segment (start 153.35 84.725) (end 153.35 89.4) (width 0.2) (layer "F.Cu") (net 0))
 (segment (start 135.625 82.65) (end 135.625 100.415) (width 0.2) (layer "F.Cu") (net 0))
 (segment (start 166.085 115.675) (end 166.085 112.475) (width 0.2) (layer "F.Cu") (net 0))
 (segment (start 174.135 89.675) (end 176.675 89.675) (width 0.2) (layer "F.Cu") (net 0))
 (segment (start 169.78376 95.938848) (end 168.911016 95.938848) (width 0.2) (layer "B.Cu") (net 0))
 (segment (start 169.877232 107.913424) (end 169.877232 104.371648) (width 0.2) (layer "B.Cu") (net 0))
 (segment (start 140.685 97.910384) (end 135.375704 92.601088) (width 0.25) (layer "B.Cu") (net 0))
 (segment (start 178.785 115.675) (end 178.854608 115.605392) (width 0.2) (layer "B.Cu") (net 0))
 (segment (start 182.119016 108.184696) (end 182.119016 108.179616) (width 0.2) (layer "B.Cu") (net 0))
 (segment (start 176.245 111.441472) (end 172.716952 107.913424) (width 0.2) (layer "B.Cu") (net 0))
 (segment (start 174.186864 85.480144) (end 176.726864 85.480144) (width 0.2) (layer "B.Cu") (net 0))
 (segment (start 128.444752 113.551208) (end 128.61544 113.38052) (width 0.25) (layer "B.Cu") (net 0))
 (segment (start 169.877232 96.03232) (end 169.78376 95.938848) (width 0.2) (layer "B.Cu") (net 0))
 (segment (start 135.375704 92.601088) (end 129.248408 92.601088) (width 0.25) (layer "B.Cu") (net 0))
 (segment (start 134.70128 108.781088) (end 134.70128 103.87872) (width 0.25) (layer "B.Cu") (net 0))
 (segment (start 135.061088 97.351088) (end 138.145 100.435) (width 0.25) (layer "B.Cu") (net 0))
 (segment (start 169.106864 85.480144) (end 171.646864 85.480144) (width 0.2) (layer "B.Cu") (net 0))
 (segment (start 172.716952 107.913424) (end 169.877232 107.913424) (width 0.2) (layer "B.Cu") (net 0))
 (segment (start 168.908984 95.936816) (end 167.108632 95.936816) (width 0.2) (layer "B.Cu") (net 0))
 (segment (start 167.108632 87.478376) (end 169.106864 85.480144) (width 0.2) (layer "B.Cu") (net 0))
 (segment (start 178.854608 111.449104) (end 182.119016 108.184696) (width 0.2) (layer "B.Cu") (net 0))
 (segment (start 128.444752 113.551208) (end 129.93116 113.551208) (width 0.25) (layer "B.Cu") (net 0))
 (segment (start 178.854608 115.605392) (end 178.854608 111.449104) (width 0.2) (layer "B.Cu") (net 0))
 (segment (start 169.877232 104.371648) (end 169.877232 96.03232) (width 0.2) (layer "B.Cu") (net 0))
 (segment (start 182.645304 91.398584) (end 176.726864 85.480144) (width 0.2) (layer "B.Cu") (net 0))
 (segment (start 176.245 115.675) (end 176.245 111.441472) (width 0.2) (layer "B.Cu") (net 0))
 (segment (start 140.685 100.435) (end 140.685 97.910384) (width 0.25) (layer "B.Cu") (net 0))
 (segment (start 168.911016 95.938848) (end 168.908984 95.936816) (width 0.2) (layer "B.Cu") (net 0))
 (segment (start 182.645304 107.653328) (end 182.645304 91.398584) (width 0.2) (layer "B.Cu") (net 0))
 (segment (start 167.108632 95.936816) (end 167.108632 87.478376) (width 0.2) (layer "B.Cu") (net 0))
 (segment (start 129.93116 113.551208) (end 134.70128 108.781088) (width 0.25) (layer "B.Cu") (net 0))
 (segment (start 182.119016 108.179616) (end 182.645304 107.653328) (width 0.2) (layer "B.Cu") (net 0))
 (segment (start 129.248408 97.351088) (end 135.061088 97.351088) (width 0.25) (layer "B.Cu") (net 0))
 (segment (start 134.70128 103.87872) (end 138.145 100.435) (width 0.25) (layer "B.Cu") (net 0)))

